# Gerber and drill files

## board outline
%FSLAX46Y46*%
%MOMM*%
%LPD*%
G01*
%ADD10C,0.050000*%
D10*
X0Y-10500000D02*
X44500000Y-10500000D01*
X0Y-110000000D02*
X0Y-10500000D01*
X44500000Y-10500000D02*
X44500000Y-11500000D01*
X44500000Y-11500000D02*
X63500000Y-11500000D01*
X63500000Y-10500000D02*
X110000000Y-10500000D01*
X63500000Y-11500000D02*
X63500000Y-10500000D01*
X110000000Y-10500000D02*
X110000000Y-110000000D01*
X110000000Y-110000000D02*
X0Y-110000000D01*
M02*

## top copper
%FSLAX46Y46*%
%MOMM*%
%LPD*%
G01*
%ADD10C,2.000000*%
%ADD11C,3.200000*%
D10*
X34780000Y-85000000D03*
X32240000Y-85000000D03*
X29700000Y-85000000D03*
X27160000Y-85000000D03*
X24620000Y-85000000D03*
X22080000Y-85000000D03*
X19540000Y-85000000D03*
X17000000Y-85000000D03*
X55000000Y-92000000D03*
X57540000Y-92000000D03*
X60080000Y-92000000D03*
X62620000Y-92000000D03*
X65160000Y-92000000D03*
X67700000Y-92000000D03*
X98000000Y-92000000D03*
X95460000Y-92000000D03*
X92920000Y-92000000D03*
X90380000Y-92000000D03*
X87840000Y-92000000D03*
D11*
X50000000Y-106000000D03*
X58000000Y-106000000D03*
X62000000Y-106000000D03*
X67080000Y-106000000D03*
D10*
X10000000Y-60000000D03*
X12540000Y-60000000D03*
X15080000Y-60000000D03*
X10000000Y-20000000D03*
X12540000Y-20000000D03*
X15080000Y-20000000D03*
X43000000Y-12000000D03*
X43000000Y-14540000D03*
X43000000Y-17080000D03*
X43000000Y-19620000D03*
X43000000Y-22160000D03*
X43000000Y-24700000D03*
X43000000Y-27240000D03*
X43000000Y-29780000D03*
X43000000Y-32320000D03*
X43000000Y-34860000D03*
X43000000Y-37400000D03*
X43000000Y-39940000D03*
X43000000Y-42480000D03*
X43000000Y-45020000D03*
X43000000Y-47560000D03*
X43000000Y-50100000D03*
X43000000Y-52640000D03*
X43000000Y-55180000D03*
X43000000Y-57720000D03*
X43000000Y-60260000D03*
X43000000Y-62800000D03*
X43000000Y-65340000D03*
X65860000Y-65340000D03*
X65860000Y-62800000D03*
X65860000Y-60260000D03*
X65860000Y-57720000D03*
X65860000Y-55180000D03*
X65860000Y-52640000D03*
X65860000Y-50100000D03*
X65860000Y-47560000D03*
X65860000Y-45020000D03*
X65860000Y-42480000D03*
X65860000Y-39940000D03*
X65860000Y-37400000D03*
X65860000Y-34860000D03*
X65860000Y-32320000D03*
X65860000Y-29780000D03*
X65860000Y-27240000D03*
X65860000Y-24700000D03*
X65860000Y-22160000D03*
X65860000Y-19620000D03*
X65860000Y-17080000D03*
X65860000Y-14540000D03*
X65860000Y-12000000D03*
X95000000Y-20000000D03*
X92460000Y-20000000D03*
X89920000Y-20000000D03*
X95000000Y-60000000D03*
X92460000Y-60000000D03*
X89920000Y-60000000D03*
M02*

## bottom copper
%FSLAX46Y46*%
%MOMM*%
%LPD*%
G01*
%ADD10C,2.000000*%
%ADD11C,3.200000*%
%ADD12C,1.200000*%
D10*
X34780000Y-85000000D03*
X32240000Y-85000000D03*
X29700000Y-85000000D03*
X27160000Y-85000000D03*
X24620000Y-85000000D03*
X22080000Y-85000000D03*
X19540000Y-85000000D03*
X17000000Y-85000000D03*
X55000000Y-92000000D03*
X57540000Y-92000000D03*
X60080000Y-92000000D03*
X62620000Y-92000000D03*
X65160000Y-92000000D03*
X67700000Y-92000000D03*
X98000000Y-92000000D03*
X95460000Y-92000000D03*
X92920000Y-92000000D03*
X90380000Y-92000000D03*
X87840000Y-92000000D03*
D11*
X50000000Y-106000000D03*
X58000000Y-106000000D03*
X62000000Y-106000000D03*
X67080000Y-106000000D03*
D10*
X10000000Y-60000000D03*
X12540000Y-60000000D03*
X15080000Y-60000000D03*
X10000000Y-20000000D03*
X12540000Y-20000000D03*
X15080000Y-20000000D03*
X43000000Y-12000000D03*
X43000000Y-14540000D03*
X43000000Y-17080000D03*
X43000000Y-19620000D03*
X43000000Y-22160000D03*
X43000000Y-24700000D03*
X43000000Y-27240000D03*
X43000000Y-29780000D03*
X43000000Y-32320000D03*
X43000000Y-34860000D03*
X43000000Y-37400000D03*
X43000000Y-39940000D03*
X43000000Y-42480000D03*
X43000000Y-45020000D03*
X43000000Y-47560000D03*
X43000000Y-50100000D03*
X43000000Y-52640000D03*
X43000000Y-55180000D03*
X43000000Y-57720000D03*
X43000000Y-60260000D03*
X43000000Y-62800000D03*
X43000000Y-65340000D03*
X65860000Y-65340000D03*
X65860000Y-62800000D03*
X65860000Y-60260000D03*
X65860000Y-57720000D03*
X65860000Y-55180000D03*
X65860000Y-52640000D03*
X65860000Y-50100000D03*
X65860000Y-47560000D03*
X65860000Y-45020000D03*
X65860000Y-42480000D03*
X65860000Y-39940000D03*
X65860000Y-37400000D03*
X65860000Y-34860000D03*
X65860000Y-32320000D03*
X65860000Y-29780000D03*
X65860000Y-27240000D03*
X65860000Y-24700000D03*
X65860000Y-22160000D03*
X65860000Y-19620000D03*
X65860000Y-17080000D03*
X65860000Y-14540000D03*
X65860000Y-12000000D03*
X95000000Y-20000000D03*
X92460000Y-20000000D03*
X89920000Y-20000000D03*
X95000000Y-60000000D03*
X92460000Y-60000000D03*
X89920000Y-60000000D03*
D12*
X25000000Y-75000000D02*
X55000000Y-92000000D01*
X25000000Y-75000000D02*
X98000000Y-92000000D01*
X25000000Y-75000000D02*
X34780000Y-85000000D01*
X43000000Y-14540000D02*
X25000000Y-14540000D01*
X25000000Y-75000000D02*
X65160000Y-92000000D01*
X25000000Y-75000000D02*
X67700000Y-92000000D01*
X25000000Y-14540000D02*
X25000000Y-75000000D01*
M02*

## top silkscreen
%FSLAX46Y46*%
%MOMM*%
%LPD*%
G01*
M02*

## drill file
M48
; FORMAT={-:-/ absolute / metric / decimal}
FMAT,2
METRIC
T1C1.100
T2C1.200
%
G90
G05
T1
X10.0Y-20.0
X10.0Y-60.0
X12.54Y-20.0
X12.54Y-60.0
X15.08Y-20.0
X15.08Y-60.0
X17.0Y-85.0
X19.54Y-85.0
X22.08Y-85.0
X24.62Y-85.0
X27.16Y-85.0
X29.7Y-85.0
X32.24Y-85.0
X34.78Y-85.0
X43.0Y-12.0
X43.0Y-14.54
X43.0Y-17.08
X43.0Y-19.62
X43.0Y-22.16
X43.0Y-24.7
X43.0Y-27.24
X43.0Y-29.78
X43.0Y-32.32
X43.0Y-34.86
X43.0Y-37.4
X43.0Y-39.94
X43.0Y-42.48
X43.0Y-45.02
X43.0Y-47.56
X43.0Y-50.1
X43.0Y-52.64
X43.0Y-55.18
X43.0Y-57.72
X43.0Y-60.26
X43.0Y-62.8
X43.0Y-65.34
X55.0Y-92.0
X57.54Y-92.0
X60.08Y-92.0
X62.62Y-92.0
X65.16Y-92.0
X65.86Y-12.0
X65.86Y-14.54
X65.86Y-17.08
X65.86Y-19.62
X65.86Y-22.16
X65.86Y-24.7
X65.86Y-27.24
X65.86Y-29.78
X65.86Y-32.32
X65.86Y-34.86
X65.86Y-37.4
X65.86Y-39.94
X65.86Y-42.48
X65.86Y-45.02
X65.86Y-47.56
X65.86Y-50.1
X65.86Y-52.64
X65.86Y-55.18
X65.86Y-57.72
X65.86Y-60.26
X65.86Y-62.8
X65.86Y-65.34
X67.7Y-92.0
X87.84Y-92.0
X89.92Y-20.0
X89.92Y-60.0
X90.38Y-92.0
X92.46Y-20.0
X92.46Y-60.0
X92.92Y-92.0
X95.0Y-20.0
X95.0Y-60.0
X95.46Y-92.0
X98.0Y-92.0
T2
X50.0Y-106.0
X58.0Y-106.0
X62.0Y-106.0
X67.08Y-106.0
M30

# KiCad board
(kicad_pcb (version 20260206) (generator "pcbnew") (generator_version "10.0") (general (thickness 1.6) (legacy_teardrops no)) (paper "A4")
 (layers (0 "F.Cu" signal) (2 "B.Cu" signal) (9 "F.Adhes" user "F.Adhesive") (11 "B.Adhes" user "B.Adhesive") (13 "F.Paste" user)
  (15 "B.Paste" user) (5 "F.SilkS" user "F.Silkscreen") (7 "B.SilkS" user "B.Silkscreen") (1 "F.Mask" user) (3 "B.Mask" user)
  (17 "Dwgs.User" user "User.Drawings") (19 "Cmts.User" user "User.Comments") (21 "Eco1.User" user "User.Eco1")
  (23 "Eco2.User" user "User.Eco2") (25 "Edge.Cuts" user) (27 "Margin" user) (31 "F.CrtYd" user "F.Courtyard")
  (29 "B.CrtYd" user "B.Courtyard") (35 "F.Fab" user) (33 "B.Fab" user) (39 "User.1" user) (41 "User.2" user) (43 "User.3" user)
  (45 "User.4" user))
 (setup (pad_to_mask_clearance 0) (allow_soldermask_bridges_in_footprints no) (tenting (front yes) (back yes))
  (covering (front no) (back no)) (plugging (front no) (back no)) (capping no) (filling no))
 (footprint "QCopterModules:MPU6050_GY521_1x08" (layer "F.Cu") (at 34.78 85 -90)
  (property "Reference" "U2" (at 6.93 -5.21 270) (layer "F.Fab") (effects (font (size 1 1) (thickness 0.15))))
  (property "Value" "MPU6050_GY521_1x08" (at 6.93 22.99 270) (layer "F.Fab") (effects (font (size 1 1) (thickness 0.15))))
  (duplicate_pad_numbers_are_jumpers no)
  (pad "1" thru_hole circle (at 0 0 270) (size 2 2) (drill 1.1) (layers "*.Cu" "*.Mask") (remove_unused_layers no) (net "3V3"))
  (pad "2" thru_hole circle (at 0 2.54 270) (size 2 2) (drill 1.1) (layers "*.Cu" "*.Mask") (remove_unused_layers no) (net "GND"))
  (pad "3" thru_hole circle (at 0 5.08 270) (size 2 2) (drill 1.1) (layers "*.Cu" "*.Mask") (remove_unused_layers no) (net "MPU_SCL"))
  (pad "4" thru_hole circle (at 0 7.62 270) (size 2 2) (drill 1.1) (layers "*.Cu" "*.Mask") (remove_unused_layers no) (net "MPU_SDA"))
  (pad "5" thru_hole circle (at 0 10.16 270) (size 2 2) (drill 1.1) (layers "*.Cu" "*.Mask") (remove_unused_layers no)
   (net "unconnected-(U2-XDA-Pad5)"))
  (pad "6" thru_hole circle (at 0 12.7 270) (size 2 2) (drill 1.1) (layers "*.Cu" "*.Mask") (remove_unused_layers no)
   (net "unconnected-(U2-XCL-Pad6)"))
  (pad "7" thru_hole circle (at 0 15.24 270) (size 2 2) (drill 1.1) (layers "*.Cu" "*.Mask") (remove_unused_layers no) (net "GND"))
  (pad "8" thru_hole circle (at 0 17.78 270) (size 2 2) (drill 1.1) (layers "*.Cu" "*.Mask") (remove_unused_layers no) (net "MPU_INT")))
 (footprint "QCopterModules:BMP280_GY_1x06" (layer "F.Cu") (at 55 92 90)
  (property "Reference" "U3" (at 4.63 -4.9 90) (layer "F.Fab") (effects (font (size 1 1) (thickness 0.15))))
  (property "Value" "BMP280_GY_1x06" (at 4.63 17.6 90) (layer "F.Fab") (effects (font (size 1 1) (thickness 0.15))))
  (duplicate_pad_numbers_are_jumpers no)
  (pad "1" thru_hole circle (at 0 0 90) (size 2 2) (drill 1.1) (layers "*.Cu" "*.Mask") (remove_unused_layers no) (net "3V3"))
  (pad "2" thru_hole circle (at 0 2.54 90) (size 2 2) (drill 1.1) (layers "*.Cu" "*.Mask") (remove_unused_layers no) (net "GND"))
  (pad "3" thru_hole circle (at 0 5.08 90) (size 2 2) (drill 1.1) (layers "*.Cu" "*.Mask") (remove_unused_layers no) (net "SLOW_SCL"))
  (pad "4" thru_hole circle (at 0 7.62 90) (size 2 2) (drill 1.1) (layers "*.Cu" "*.Mask") (remove_unused_layers no) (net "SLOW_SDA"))
  (pad "5" thru_hole circle (at 0 10.16 90) (size 2 2) (drill 1.1) (layers "*.Cu" "*.Mask") (remove_unused_layers no) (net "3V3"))
  (pad "6" thru_hole circle (at 0 12.7 90) (size 2 2) (drill 1.1) (layers "*.Cu" "*.Mask") (remove_unused_layers no) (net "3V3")))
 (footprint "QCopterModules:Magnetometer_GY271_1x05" (layer "F.Cu") (at 98 92 -90)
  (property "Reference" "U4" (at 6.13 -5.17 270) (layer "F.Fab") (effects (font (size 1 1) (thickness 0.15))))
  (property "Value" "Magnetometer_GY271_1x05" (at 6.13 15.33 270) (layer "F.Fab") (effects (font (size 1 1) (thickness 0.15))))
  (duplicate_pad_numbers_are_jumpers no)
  (pad "1" thru_hole circle (at 0 0 270) (size 2 2) (drill 1.1) (layers "*.Cu" "*.Mask") (remove_unused_layers no) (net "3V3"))
  (pad "2" thru_hole circle (at 0 2.54 270) (size 2 2) (drill 1.1) (layers "*.Cu" "*.Mask") (remove_unused_layers no) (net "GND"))
  (pad "3" thru_hole circle (at 0 5.08 270) (size 2 2) (drill 1.1) (layers "*.Cu" "*.Mask") (remove_unused_layers no) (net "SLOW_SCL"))
  (pad "4" thru_hole circle (at 0 7.62 270) (size 2 2) (drill 1.1) (layers "*.Cu" "*.Mask") (remove_unused_layers no) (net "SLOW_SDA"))
  (pad "5" thru_hole circle (at 0 10.16 270) (size 2 2) (drill 1.1) (layers "*.Cu" "*.Mask") (remove_unused_layers no) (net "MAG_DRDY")))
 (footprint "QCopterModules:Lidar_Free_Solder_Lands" (layer "F.Cu") (at 50 106)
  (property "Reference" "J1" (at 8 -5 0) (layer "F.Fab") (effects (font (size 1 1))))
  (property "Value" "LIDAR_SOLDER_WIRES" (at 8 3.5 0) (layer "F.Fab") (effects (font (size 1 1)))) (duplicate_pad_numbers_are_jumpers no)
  (pad "1" thru_hole circle (at 0 0) (size 3.2 3.2) (drill 1.2) (layers "*.Cu" "*.Mask") (remove_unused_layers no) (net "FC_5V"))
  (pad "2" thru_hole circle (at 8 0) (size 3.2 3.2) (drill 1.2) (layers "*.Cu" "*.Mask") (remove_unused_layers no) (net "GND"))
  (pad "3" thru_hole circle (at 12 0) (size 3.2 3.2) (drill 1.2) (layers "*.Cu" "*.Mask") (remove_unused_layers no) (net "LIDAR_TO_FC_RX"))
  (pad "4" thru_hole circle (at 17.08 0) (size 3.2 3.2) (drill 1.2) (layers "*.Cu" "*.Mask") (remove_unused_layers no)
   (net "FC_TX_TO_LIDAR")))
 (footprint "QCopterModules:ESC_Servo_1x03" (layer "F.Cu") (at 10 60 90)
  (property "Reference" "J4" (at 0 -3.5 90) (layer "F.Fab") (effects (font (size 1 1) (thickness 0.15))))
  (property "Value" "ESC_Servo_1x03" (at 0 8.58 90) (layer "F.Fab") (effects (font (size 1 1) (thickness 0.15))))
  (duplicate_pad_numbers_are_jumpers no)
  (pad "1" thru_hole circle (at 0 0 90) (size 2 2) (drill 1.1) (layers "*.Cu" "*.Mask") (remove_unused_layers no) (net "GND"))
  (pad "2" thru_hole circle (at 0 2.54 90) (size 2 2) (drill 1.1) (layers "*.Cu" "*.Mask") (remove_unused_layers no) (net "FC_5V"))
  (pad "3" thru_hole circle (at 0 5.08 90) (size 2 2) (drill 1.1) (layers "*.Cu" "*.Mask") (remove_unused_layers no) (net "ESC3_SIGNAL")))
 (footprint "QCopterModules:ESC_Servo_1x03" (layer "F.Cu") (at 10 20 90)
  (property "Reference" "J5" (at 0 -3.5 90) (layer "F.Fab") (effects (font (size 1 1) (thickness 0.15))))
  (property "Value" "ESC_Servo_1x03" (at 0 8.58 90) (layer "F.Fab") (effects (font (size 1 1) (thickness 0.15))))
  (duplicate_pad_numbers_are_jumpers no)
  (pad "1" thru_hole circle (at 0 0 90) (size 2 2) (drill 1.1) (layers "*.Cu" "*.Mask") (remove_unused_layers no) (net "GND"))
  (pad "2" thru_hole circle (at 0 2.54 90) (size 2 2) (drill 1.1) (layers "*.Cu" "*.Mask") (remove_unused_layers no)
   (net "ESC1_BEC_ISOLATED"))
  (pad "3" thru_hole circle (at 0 5.08 90) (size 2 2) (drill 1.1) (layers "*.Cu" "*.Mask") (remove_unused_layers no) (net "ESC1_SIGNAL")))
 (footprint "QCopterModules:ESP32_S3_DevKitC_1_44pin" (layer "F.Cu") (at 43 12)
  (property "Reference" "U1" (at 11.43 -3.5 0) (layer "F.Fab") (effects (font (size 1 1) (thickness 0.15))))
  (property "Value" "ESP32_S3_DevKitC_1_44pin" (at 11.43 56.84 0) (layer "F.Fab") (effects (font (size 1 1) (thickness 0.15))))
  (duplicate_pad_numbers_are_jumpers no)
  (pad "1" thru_hole circle (at 0 0) (size 2 2) (drill 1.1) (layers "*.Cu" "*.Mask") (remove_unused_layers no))
  (pad "2" thru_hole circle (at 0 2.54) (size 2 2) (drill 1.1) (layers "*.Cu" "*.Mask") (remove_unused_layers no) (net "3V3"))
  (pad "3" thru_hole circle (at 0 5.08) (size 2 2) (drill 1.1) (layers "*.Cu" "*.Mask") (remove_unused_layers no)
   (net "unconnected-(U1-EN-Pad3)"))
  (pad "4" thru_hole circle (at 0 7.62) (size 2 2) (drill 1.1) (layers "*.Cu" "*.Mask") (remove_unused_layers no) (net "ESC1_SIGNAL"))
  (pad "5" thru_hole circle (at 0 10.16) (size 2 2) (drill 1.1) (layers "*.Cu" "*.Mask") (remove_unused_layers no)
   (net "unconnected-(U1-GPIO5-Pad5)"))
  (pad "6" thru_hole circle (at 0 12.7) (size 2 2) (drill 1.1) (layers "*.Cu" "*.Mask") (remove_unused_layers no)
   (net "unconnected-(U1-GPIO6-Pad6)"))
  (pad "7" thru_hole circle (at 0 15.24) (size 2 2) (drill 1.1) (layers "*.Cu" "*.Mask") (remove_unused_layers no)
   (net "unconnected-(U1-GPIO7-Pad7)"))
  (pad "8" thru_hole circle (at 0 17.78) (size 2 2) (drill 1.1) (layers "*.Cu" "*.Mask") (remove_unused_layers no) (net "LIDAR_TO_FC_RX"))
  (pad "9" thru_hole circle (at 0 20.32) (size 2 2) (drill 1.1) (layers "*.Cu" "*.Mask") (remove_unused_layers no) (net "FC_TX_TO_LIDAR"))
  (pad "10" thru_hole circle (at 0 22.86) (size 2 2) (drill 1.1) (layers "*.Cu" "*.Mask") (remove_unused_layers no)
   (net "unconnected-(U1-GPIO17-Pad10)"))
  (pad "11" thru_hole circle (at 0 25.4) (size 2 2) (drill 1.1) (layers "*.Cu" "*.Mask") (remove_unused_layers no) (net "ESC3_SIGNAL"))
  (pad "12" thru_hole circle (at 0 27.94) (size 2 2) (drill 1.1) (layers "*.Cu" "*.Mask") (remove_unused_layers no)
   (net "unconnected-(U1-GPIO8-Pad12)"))
  (pad "13" thru_hole circle (at 0 30.48) (size 2 2) (drill 1.1) (layers "*.Cu" "*.Mask") (remove_unused_layers no)
   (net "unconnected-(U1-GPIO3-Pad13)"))
  (pad "14" thru_hole circle (at 0 33.02) (size 2 2) (drill 1.1) (layers "*.Cu" "*.Mask") (remove_unused_layers no)
   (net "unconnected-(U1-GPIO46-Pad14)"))
  (pad "15" thru_hole circle (at 0 35.56) (size 2 2) (drill 1.1) (layers "*.Cu" "*.Mask") (remove_unused_layers no)
   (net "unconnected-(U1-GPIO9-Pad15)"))
  (pad "16" thru_hole circle (at 0 38.1) (size 2 2) (drill 1.1) (layers "*.Cu" "*.Mask") (remove_unused_layers no)
   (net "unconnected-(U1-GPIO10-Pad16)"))
  (pad "17" thru_hole circle (at 0 40.64) (size 2 2) (drill 1.1) (layers "*.Cu" "*.Mask") (remove_unused_layers no)
   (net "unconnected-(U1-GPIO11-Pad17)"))
  (pad "18" thru_hole circle (at 0 43.18) (size 2 2) (drill 1.1) (layers "*.Cu" "*.Mask") (remove_unused_layers no) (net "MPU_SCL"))
  (pad "19" thru_hole circle (at 0 45.72) (size 2 2) (drill 1.1) (layers "*.Cu" "*.Mask") (remove_unused_layers no) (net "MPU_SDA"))
  (pad "20" thru_hole circle (at 0 48.26) (size 2 2) (drill 1.1) (layers "*.Cu" "*.Mask") (remove_unused_layers no) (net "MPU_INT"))
  (pad "21" thru_hole circle (at 0 50.8) (size 2 2) (drill 1.1) (layers "*.Cu" "*.Mask") (remove_unused_layers no) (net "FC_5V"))
  (pad "22" thru_hole circle (at 0 53.34) (size 2 2) (drill 1.1) (layers "*.Cu" "*.Mask") (remove_unused_layers no) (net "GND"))
  (pad "23" thru_hole circle (at 22.86 53.34) (size 2 2) (drill 1.1) (layers "*.Cu" "*.Mask") (remove_unused_layers no) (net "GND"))
  (pad "24" thru_hole circle (at 22.86 50.8) (size 2 2) (drill 1.1) (layers "*.Cu" "*.Mask") (remove_unused_layers no) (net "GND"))
  (pad "25" thru_hole circle (at 22.86 48.26) (size 2 2) (drill 1.1) (layers "*.Cu" "*.Mask") (remove_unused_layers no)
   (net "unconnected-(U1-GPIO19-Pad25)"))
  (pad "26" thru_hole circle (at 22.86 45.72) (size 2 2) (drill 1.1) (layers "*.Cu" "*.Mask") (remove_unused_layers no)
   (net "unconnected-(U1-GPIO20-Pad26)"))
  (pad "27" thru_hole circle (at 22.86 43.18) (size 2 2) (drill 1.1) (layers "*.Cu" "*.Mask") (remove_unused_layers no) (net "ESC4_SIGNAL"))
  (pad "28" thru_hole circle (at 22.86 40.64) (size 2 2) (drill 1.1) (layers "*.Cu" "*.Mask") (remove_unused_layers no)
   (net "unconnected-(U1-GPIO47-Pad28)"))
  (pad "29" thru_hole circle (at 22.86 38.1) (size 2 2) (drill 1.1) (layers "*.Cu" "*.Mask") (remove_unused_layers no)
   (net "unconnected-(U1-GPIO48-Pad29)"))
  (pad "30" thru_hole circle (at 22.86 35.56) (size 2 2) (drill 1.1) (layers "*.Cu" "*.Mask") (remove_unused_layers no)
   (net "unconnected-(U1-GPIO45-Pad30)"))
  (pad "31" thru_hole circle (at 22.86 33.02) (size 2 2) (drill 1.1) (layers "*.Cu" "*.Mask") (remove_unused_layers no)
   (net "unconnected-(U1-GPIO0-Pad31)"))
  (pad "32" thru_hole circle (at 22.86 30.48) (size 2 2) (drill 1.1) (layers "*.Cu" "*.Mask") (remove_unused_layers no)
   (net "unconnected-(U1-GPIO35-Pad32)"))
  (pad "33" thru_hole circle (at 22.86 27.94) (size 2 2) (drill 1.1) (layers "*.Cu" "*.Mask") (remove_unused_layers no)
   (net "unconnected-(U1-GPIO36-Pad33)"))
  (pad "34" thru_hole circle (at 22.86 25.4) (size 2 2) (drill 1.1) (layers "*.Cu" "*.Mask") (remove_unused_layers no)
   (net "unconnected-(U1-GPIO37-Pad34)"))
  (pad "35" thru_hole circle (at 22.86 22.86) (size 2 2) (drill 1.1) (layers "*.Cu" "*.Mask") (remove_unused_layers no)
   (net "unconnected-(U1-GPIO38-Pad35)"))
  (pad "36" thru_hole circle (at 22.86 20.32) (size 2 2) (drill 1.1) (layers "*.Cu" "*.Mask") (remove_unused_layers no) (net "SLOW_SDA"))
  (pad "37" thru_hole circle (at 22.86 17.78) (size 2 2) (drill 1.1) (layers "*.Cu" "*.Mask") (remove_unused_layers no) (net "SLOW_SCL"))
  (pad "38" thru_hole circle (at 22.86 15.24) (size 2 2) (drill 1.1) (layers "*.Cu" "*.Mask") (remove_unused_layers no) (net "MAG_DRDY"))
  (pad "39" thru_hole circle (at 22.86 12.7) (size 2 2) (drill 1.1) (layers "*.Cu" "*.Mask") (remove_unused_layers no)
   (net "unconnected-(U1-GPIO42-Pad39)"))
  (pad "40" thru_hole circle (at 22.86 10.16) (size 2 2) (drill 1.1) (layers "*.Cu" "*.Mask") (remove_unused_layers no) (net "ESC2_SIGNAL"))
  (pad "41" thru_hole circle (at 22.86 7.62) (size 2 2) (drill 1.1) (layers "*.Cu" "*.Mask") (remove_unused_layers no)
   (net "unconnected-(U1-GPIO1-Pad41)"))
  (pad "42" thru_hole circle (at 22.86 5.08) (size 2 2) (drill 1.1) (layers "*.Cu" "*.Mask") (remove_unused_layers no)
   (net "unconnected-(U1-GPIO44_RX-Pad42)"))
  (pad "43" thru_hole circle (at 22.86 2.54) (size 2 2) (drill 1.1) (layers "*.Cu" "*.Mask") (remove_unused_layers no)
   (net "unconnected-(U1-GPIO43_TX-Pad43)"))
  (pad "44" thru_hole circle (at 22.86 0) (size 2 2) (drill 1.1) (layers "*.Cu" "*.Mask") (remove_unused_layers no) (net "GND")))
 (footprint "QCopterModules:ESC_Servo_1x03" (layer "F.Cu") (at 95 20 -90)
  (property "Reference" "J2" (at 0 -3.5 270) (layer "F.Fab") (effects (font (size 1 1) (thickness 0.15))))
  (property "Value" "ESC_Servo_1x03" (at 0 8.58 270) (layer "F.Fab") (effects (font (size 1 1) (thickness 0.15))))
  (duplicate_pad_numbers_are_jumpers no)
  (pad "1" thru_hole circle (at 0 0 270) (size 2 2) (drill 1.1) (layers "*.Cu" "*.Mask") (remove_unused_layers no) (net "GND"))
  (pad "2" thru_hole circle (at 0 2.54 270) (size 2 2) (drill 1.1) (layers "*.Cu" "*.Mask") (remove_unused_layers no)
   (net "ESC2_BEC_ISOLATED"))
  (pad "3" thru_hole circle (at 0 5.08 270) (size 2 2) (drill 1.1) (layers "*.Cu" "*.Mask") (remove_unused_layers no) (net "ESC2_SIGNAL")))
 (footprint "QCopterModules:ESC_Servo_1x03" (layer "F.Cu") (at 95 60 -90)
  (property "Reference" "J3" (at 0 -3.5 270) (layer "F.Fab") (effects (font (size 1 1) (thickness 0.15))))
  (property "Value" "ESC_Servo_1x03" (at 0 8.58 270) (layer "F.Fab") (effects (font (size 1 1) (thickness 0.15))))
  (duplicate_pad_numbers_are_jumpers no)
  (pad "1" thru_hole circle (at 0 0 270) (size 2 2) (drill 1.1) (layers "*.Cu" "*.Mask") (remove_unused_layers no) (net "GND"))
  (pad "2" thru_hole circle (at 0 2.54 270) (size 2 2) (drill 1.1) (layers "*.Cu" "*.Mask") (remove_unused_layers no)
   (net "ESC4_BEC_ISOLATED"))
  (pad "3" thru_hole circle (at 0 5.08 270) (size 2 2) (drill 1.1) (layers "*.Cu" "*.Mask") (remove_unused_layers no) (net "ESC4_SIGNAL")))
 (gr_line (start 0 10.5) (end 44.5 10.5) (stroke (width 0.05) (type default)) (layer "Edge.Cuts"))
 (gr_line (start 0 110) (end 0 10.5) (stroke (width 0.05) (type default)) (layer "Edge.Cuts"))
 (gr_line (start 44.5 10.5) (end 44.5 11.5) (stroke (width 0.05) (type default)) (layer "Edge.Cuts"))
 (gr_line (start 44.5 11.5) (end 63.5 11.5) (stroke (width 0.05) (type default)) (layer "Edge.Cuts"))
 (gr_line (start 63.5 10.5) (end 110 10.5) (stroke (width 0.05) (type default)) (layer "Edge.Cuts"))
 (gr_line (start 63.5 11.5) (end 63.5 10.5) (stroke (width 0.05) (type default)) (layer "Edge.Cuts"))
 (gr_line (start 110 10.5) (end 110 110) (stroke (width 0.05) (type default)) (layer "Edge.Cuts"))
 (gr_line (start 110 110) (end 0 110) (stroke (width 0.05) (type default)) (layer "Edge.Cuts"))
 (segment (start 25 75) (end 55 92) (width 1.2) (layer "B.Cu") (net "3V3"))
 (segment (start 25 75) (end 98 92) (width 1.2) (layer "B.Cu") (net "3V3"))
 (segment (start 25 75) (end 34.78 85) (width 1.2) (layer "B.Cu") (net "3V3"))
 (segment (start 43 14.54) (end 25 14.54) (width 1.2) (layer "B.Cu") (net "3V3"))
 (segment (start 25 75) (end 65.16 92) (width 1.2) (layer "B.Cu") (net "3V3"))
 (segment (start 25 75) (end 67.7 92) (width 1.2) (layer "B.Cu") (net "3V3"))
 (segment (start 25 14.54) (end 25 75) (width 1.2) (layer "B.Cu") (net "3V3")))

